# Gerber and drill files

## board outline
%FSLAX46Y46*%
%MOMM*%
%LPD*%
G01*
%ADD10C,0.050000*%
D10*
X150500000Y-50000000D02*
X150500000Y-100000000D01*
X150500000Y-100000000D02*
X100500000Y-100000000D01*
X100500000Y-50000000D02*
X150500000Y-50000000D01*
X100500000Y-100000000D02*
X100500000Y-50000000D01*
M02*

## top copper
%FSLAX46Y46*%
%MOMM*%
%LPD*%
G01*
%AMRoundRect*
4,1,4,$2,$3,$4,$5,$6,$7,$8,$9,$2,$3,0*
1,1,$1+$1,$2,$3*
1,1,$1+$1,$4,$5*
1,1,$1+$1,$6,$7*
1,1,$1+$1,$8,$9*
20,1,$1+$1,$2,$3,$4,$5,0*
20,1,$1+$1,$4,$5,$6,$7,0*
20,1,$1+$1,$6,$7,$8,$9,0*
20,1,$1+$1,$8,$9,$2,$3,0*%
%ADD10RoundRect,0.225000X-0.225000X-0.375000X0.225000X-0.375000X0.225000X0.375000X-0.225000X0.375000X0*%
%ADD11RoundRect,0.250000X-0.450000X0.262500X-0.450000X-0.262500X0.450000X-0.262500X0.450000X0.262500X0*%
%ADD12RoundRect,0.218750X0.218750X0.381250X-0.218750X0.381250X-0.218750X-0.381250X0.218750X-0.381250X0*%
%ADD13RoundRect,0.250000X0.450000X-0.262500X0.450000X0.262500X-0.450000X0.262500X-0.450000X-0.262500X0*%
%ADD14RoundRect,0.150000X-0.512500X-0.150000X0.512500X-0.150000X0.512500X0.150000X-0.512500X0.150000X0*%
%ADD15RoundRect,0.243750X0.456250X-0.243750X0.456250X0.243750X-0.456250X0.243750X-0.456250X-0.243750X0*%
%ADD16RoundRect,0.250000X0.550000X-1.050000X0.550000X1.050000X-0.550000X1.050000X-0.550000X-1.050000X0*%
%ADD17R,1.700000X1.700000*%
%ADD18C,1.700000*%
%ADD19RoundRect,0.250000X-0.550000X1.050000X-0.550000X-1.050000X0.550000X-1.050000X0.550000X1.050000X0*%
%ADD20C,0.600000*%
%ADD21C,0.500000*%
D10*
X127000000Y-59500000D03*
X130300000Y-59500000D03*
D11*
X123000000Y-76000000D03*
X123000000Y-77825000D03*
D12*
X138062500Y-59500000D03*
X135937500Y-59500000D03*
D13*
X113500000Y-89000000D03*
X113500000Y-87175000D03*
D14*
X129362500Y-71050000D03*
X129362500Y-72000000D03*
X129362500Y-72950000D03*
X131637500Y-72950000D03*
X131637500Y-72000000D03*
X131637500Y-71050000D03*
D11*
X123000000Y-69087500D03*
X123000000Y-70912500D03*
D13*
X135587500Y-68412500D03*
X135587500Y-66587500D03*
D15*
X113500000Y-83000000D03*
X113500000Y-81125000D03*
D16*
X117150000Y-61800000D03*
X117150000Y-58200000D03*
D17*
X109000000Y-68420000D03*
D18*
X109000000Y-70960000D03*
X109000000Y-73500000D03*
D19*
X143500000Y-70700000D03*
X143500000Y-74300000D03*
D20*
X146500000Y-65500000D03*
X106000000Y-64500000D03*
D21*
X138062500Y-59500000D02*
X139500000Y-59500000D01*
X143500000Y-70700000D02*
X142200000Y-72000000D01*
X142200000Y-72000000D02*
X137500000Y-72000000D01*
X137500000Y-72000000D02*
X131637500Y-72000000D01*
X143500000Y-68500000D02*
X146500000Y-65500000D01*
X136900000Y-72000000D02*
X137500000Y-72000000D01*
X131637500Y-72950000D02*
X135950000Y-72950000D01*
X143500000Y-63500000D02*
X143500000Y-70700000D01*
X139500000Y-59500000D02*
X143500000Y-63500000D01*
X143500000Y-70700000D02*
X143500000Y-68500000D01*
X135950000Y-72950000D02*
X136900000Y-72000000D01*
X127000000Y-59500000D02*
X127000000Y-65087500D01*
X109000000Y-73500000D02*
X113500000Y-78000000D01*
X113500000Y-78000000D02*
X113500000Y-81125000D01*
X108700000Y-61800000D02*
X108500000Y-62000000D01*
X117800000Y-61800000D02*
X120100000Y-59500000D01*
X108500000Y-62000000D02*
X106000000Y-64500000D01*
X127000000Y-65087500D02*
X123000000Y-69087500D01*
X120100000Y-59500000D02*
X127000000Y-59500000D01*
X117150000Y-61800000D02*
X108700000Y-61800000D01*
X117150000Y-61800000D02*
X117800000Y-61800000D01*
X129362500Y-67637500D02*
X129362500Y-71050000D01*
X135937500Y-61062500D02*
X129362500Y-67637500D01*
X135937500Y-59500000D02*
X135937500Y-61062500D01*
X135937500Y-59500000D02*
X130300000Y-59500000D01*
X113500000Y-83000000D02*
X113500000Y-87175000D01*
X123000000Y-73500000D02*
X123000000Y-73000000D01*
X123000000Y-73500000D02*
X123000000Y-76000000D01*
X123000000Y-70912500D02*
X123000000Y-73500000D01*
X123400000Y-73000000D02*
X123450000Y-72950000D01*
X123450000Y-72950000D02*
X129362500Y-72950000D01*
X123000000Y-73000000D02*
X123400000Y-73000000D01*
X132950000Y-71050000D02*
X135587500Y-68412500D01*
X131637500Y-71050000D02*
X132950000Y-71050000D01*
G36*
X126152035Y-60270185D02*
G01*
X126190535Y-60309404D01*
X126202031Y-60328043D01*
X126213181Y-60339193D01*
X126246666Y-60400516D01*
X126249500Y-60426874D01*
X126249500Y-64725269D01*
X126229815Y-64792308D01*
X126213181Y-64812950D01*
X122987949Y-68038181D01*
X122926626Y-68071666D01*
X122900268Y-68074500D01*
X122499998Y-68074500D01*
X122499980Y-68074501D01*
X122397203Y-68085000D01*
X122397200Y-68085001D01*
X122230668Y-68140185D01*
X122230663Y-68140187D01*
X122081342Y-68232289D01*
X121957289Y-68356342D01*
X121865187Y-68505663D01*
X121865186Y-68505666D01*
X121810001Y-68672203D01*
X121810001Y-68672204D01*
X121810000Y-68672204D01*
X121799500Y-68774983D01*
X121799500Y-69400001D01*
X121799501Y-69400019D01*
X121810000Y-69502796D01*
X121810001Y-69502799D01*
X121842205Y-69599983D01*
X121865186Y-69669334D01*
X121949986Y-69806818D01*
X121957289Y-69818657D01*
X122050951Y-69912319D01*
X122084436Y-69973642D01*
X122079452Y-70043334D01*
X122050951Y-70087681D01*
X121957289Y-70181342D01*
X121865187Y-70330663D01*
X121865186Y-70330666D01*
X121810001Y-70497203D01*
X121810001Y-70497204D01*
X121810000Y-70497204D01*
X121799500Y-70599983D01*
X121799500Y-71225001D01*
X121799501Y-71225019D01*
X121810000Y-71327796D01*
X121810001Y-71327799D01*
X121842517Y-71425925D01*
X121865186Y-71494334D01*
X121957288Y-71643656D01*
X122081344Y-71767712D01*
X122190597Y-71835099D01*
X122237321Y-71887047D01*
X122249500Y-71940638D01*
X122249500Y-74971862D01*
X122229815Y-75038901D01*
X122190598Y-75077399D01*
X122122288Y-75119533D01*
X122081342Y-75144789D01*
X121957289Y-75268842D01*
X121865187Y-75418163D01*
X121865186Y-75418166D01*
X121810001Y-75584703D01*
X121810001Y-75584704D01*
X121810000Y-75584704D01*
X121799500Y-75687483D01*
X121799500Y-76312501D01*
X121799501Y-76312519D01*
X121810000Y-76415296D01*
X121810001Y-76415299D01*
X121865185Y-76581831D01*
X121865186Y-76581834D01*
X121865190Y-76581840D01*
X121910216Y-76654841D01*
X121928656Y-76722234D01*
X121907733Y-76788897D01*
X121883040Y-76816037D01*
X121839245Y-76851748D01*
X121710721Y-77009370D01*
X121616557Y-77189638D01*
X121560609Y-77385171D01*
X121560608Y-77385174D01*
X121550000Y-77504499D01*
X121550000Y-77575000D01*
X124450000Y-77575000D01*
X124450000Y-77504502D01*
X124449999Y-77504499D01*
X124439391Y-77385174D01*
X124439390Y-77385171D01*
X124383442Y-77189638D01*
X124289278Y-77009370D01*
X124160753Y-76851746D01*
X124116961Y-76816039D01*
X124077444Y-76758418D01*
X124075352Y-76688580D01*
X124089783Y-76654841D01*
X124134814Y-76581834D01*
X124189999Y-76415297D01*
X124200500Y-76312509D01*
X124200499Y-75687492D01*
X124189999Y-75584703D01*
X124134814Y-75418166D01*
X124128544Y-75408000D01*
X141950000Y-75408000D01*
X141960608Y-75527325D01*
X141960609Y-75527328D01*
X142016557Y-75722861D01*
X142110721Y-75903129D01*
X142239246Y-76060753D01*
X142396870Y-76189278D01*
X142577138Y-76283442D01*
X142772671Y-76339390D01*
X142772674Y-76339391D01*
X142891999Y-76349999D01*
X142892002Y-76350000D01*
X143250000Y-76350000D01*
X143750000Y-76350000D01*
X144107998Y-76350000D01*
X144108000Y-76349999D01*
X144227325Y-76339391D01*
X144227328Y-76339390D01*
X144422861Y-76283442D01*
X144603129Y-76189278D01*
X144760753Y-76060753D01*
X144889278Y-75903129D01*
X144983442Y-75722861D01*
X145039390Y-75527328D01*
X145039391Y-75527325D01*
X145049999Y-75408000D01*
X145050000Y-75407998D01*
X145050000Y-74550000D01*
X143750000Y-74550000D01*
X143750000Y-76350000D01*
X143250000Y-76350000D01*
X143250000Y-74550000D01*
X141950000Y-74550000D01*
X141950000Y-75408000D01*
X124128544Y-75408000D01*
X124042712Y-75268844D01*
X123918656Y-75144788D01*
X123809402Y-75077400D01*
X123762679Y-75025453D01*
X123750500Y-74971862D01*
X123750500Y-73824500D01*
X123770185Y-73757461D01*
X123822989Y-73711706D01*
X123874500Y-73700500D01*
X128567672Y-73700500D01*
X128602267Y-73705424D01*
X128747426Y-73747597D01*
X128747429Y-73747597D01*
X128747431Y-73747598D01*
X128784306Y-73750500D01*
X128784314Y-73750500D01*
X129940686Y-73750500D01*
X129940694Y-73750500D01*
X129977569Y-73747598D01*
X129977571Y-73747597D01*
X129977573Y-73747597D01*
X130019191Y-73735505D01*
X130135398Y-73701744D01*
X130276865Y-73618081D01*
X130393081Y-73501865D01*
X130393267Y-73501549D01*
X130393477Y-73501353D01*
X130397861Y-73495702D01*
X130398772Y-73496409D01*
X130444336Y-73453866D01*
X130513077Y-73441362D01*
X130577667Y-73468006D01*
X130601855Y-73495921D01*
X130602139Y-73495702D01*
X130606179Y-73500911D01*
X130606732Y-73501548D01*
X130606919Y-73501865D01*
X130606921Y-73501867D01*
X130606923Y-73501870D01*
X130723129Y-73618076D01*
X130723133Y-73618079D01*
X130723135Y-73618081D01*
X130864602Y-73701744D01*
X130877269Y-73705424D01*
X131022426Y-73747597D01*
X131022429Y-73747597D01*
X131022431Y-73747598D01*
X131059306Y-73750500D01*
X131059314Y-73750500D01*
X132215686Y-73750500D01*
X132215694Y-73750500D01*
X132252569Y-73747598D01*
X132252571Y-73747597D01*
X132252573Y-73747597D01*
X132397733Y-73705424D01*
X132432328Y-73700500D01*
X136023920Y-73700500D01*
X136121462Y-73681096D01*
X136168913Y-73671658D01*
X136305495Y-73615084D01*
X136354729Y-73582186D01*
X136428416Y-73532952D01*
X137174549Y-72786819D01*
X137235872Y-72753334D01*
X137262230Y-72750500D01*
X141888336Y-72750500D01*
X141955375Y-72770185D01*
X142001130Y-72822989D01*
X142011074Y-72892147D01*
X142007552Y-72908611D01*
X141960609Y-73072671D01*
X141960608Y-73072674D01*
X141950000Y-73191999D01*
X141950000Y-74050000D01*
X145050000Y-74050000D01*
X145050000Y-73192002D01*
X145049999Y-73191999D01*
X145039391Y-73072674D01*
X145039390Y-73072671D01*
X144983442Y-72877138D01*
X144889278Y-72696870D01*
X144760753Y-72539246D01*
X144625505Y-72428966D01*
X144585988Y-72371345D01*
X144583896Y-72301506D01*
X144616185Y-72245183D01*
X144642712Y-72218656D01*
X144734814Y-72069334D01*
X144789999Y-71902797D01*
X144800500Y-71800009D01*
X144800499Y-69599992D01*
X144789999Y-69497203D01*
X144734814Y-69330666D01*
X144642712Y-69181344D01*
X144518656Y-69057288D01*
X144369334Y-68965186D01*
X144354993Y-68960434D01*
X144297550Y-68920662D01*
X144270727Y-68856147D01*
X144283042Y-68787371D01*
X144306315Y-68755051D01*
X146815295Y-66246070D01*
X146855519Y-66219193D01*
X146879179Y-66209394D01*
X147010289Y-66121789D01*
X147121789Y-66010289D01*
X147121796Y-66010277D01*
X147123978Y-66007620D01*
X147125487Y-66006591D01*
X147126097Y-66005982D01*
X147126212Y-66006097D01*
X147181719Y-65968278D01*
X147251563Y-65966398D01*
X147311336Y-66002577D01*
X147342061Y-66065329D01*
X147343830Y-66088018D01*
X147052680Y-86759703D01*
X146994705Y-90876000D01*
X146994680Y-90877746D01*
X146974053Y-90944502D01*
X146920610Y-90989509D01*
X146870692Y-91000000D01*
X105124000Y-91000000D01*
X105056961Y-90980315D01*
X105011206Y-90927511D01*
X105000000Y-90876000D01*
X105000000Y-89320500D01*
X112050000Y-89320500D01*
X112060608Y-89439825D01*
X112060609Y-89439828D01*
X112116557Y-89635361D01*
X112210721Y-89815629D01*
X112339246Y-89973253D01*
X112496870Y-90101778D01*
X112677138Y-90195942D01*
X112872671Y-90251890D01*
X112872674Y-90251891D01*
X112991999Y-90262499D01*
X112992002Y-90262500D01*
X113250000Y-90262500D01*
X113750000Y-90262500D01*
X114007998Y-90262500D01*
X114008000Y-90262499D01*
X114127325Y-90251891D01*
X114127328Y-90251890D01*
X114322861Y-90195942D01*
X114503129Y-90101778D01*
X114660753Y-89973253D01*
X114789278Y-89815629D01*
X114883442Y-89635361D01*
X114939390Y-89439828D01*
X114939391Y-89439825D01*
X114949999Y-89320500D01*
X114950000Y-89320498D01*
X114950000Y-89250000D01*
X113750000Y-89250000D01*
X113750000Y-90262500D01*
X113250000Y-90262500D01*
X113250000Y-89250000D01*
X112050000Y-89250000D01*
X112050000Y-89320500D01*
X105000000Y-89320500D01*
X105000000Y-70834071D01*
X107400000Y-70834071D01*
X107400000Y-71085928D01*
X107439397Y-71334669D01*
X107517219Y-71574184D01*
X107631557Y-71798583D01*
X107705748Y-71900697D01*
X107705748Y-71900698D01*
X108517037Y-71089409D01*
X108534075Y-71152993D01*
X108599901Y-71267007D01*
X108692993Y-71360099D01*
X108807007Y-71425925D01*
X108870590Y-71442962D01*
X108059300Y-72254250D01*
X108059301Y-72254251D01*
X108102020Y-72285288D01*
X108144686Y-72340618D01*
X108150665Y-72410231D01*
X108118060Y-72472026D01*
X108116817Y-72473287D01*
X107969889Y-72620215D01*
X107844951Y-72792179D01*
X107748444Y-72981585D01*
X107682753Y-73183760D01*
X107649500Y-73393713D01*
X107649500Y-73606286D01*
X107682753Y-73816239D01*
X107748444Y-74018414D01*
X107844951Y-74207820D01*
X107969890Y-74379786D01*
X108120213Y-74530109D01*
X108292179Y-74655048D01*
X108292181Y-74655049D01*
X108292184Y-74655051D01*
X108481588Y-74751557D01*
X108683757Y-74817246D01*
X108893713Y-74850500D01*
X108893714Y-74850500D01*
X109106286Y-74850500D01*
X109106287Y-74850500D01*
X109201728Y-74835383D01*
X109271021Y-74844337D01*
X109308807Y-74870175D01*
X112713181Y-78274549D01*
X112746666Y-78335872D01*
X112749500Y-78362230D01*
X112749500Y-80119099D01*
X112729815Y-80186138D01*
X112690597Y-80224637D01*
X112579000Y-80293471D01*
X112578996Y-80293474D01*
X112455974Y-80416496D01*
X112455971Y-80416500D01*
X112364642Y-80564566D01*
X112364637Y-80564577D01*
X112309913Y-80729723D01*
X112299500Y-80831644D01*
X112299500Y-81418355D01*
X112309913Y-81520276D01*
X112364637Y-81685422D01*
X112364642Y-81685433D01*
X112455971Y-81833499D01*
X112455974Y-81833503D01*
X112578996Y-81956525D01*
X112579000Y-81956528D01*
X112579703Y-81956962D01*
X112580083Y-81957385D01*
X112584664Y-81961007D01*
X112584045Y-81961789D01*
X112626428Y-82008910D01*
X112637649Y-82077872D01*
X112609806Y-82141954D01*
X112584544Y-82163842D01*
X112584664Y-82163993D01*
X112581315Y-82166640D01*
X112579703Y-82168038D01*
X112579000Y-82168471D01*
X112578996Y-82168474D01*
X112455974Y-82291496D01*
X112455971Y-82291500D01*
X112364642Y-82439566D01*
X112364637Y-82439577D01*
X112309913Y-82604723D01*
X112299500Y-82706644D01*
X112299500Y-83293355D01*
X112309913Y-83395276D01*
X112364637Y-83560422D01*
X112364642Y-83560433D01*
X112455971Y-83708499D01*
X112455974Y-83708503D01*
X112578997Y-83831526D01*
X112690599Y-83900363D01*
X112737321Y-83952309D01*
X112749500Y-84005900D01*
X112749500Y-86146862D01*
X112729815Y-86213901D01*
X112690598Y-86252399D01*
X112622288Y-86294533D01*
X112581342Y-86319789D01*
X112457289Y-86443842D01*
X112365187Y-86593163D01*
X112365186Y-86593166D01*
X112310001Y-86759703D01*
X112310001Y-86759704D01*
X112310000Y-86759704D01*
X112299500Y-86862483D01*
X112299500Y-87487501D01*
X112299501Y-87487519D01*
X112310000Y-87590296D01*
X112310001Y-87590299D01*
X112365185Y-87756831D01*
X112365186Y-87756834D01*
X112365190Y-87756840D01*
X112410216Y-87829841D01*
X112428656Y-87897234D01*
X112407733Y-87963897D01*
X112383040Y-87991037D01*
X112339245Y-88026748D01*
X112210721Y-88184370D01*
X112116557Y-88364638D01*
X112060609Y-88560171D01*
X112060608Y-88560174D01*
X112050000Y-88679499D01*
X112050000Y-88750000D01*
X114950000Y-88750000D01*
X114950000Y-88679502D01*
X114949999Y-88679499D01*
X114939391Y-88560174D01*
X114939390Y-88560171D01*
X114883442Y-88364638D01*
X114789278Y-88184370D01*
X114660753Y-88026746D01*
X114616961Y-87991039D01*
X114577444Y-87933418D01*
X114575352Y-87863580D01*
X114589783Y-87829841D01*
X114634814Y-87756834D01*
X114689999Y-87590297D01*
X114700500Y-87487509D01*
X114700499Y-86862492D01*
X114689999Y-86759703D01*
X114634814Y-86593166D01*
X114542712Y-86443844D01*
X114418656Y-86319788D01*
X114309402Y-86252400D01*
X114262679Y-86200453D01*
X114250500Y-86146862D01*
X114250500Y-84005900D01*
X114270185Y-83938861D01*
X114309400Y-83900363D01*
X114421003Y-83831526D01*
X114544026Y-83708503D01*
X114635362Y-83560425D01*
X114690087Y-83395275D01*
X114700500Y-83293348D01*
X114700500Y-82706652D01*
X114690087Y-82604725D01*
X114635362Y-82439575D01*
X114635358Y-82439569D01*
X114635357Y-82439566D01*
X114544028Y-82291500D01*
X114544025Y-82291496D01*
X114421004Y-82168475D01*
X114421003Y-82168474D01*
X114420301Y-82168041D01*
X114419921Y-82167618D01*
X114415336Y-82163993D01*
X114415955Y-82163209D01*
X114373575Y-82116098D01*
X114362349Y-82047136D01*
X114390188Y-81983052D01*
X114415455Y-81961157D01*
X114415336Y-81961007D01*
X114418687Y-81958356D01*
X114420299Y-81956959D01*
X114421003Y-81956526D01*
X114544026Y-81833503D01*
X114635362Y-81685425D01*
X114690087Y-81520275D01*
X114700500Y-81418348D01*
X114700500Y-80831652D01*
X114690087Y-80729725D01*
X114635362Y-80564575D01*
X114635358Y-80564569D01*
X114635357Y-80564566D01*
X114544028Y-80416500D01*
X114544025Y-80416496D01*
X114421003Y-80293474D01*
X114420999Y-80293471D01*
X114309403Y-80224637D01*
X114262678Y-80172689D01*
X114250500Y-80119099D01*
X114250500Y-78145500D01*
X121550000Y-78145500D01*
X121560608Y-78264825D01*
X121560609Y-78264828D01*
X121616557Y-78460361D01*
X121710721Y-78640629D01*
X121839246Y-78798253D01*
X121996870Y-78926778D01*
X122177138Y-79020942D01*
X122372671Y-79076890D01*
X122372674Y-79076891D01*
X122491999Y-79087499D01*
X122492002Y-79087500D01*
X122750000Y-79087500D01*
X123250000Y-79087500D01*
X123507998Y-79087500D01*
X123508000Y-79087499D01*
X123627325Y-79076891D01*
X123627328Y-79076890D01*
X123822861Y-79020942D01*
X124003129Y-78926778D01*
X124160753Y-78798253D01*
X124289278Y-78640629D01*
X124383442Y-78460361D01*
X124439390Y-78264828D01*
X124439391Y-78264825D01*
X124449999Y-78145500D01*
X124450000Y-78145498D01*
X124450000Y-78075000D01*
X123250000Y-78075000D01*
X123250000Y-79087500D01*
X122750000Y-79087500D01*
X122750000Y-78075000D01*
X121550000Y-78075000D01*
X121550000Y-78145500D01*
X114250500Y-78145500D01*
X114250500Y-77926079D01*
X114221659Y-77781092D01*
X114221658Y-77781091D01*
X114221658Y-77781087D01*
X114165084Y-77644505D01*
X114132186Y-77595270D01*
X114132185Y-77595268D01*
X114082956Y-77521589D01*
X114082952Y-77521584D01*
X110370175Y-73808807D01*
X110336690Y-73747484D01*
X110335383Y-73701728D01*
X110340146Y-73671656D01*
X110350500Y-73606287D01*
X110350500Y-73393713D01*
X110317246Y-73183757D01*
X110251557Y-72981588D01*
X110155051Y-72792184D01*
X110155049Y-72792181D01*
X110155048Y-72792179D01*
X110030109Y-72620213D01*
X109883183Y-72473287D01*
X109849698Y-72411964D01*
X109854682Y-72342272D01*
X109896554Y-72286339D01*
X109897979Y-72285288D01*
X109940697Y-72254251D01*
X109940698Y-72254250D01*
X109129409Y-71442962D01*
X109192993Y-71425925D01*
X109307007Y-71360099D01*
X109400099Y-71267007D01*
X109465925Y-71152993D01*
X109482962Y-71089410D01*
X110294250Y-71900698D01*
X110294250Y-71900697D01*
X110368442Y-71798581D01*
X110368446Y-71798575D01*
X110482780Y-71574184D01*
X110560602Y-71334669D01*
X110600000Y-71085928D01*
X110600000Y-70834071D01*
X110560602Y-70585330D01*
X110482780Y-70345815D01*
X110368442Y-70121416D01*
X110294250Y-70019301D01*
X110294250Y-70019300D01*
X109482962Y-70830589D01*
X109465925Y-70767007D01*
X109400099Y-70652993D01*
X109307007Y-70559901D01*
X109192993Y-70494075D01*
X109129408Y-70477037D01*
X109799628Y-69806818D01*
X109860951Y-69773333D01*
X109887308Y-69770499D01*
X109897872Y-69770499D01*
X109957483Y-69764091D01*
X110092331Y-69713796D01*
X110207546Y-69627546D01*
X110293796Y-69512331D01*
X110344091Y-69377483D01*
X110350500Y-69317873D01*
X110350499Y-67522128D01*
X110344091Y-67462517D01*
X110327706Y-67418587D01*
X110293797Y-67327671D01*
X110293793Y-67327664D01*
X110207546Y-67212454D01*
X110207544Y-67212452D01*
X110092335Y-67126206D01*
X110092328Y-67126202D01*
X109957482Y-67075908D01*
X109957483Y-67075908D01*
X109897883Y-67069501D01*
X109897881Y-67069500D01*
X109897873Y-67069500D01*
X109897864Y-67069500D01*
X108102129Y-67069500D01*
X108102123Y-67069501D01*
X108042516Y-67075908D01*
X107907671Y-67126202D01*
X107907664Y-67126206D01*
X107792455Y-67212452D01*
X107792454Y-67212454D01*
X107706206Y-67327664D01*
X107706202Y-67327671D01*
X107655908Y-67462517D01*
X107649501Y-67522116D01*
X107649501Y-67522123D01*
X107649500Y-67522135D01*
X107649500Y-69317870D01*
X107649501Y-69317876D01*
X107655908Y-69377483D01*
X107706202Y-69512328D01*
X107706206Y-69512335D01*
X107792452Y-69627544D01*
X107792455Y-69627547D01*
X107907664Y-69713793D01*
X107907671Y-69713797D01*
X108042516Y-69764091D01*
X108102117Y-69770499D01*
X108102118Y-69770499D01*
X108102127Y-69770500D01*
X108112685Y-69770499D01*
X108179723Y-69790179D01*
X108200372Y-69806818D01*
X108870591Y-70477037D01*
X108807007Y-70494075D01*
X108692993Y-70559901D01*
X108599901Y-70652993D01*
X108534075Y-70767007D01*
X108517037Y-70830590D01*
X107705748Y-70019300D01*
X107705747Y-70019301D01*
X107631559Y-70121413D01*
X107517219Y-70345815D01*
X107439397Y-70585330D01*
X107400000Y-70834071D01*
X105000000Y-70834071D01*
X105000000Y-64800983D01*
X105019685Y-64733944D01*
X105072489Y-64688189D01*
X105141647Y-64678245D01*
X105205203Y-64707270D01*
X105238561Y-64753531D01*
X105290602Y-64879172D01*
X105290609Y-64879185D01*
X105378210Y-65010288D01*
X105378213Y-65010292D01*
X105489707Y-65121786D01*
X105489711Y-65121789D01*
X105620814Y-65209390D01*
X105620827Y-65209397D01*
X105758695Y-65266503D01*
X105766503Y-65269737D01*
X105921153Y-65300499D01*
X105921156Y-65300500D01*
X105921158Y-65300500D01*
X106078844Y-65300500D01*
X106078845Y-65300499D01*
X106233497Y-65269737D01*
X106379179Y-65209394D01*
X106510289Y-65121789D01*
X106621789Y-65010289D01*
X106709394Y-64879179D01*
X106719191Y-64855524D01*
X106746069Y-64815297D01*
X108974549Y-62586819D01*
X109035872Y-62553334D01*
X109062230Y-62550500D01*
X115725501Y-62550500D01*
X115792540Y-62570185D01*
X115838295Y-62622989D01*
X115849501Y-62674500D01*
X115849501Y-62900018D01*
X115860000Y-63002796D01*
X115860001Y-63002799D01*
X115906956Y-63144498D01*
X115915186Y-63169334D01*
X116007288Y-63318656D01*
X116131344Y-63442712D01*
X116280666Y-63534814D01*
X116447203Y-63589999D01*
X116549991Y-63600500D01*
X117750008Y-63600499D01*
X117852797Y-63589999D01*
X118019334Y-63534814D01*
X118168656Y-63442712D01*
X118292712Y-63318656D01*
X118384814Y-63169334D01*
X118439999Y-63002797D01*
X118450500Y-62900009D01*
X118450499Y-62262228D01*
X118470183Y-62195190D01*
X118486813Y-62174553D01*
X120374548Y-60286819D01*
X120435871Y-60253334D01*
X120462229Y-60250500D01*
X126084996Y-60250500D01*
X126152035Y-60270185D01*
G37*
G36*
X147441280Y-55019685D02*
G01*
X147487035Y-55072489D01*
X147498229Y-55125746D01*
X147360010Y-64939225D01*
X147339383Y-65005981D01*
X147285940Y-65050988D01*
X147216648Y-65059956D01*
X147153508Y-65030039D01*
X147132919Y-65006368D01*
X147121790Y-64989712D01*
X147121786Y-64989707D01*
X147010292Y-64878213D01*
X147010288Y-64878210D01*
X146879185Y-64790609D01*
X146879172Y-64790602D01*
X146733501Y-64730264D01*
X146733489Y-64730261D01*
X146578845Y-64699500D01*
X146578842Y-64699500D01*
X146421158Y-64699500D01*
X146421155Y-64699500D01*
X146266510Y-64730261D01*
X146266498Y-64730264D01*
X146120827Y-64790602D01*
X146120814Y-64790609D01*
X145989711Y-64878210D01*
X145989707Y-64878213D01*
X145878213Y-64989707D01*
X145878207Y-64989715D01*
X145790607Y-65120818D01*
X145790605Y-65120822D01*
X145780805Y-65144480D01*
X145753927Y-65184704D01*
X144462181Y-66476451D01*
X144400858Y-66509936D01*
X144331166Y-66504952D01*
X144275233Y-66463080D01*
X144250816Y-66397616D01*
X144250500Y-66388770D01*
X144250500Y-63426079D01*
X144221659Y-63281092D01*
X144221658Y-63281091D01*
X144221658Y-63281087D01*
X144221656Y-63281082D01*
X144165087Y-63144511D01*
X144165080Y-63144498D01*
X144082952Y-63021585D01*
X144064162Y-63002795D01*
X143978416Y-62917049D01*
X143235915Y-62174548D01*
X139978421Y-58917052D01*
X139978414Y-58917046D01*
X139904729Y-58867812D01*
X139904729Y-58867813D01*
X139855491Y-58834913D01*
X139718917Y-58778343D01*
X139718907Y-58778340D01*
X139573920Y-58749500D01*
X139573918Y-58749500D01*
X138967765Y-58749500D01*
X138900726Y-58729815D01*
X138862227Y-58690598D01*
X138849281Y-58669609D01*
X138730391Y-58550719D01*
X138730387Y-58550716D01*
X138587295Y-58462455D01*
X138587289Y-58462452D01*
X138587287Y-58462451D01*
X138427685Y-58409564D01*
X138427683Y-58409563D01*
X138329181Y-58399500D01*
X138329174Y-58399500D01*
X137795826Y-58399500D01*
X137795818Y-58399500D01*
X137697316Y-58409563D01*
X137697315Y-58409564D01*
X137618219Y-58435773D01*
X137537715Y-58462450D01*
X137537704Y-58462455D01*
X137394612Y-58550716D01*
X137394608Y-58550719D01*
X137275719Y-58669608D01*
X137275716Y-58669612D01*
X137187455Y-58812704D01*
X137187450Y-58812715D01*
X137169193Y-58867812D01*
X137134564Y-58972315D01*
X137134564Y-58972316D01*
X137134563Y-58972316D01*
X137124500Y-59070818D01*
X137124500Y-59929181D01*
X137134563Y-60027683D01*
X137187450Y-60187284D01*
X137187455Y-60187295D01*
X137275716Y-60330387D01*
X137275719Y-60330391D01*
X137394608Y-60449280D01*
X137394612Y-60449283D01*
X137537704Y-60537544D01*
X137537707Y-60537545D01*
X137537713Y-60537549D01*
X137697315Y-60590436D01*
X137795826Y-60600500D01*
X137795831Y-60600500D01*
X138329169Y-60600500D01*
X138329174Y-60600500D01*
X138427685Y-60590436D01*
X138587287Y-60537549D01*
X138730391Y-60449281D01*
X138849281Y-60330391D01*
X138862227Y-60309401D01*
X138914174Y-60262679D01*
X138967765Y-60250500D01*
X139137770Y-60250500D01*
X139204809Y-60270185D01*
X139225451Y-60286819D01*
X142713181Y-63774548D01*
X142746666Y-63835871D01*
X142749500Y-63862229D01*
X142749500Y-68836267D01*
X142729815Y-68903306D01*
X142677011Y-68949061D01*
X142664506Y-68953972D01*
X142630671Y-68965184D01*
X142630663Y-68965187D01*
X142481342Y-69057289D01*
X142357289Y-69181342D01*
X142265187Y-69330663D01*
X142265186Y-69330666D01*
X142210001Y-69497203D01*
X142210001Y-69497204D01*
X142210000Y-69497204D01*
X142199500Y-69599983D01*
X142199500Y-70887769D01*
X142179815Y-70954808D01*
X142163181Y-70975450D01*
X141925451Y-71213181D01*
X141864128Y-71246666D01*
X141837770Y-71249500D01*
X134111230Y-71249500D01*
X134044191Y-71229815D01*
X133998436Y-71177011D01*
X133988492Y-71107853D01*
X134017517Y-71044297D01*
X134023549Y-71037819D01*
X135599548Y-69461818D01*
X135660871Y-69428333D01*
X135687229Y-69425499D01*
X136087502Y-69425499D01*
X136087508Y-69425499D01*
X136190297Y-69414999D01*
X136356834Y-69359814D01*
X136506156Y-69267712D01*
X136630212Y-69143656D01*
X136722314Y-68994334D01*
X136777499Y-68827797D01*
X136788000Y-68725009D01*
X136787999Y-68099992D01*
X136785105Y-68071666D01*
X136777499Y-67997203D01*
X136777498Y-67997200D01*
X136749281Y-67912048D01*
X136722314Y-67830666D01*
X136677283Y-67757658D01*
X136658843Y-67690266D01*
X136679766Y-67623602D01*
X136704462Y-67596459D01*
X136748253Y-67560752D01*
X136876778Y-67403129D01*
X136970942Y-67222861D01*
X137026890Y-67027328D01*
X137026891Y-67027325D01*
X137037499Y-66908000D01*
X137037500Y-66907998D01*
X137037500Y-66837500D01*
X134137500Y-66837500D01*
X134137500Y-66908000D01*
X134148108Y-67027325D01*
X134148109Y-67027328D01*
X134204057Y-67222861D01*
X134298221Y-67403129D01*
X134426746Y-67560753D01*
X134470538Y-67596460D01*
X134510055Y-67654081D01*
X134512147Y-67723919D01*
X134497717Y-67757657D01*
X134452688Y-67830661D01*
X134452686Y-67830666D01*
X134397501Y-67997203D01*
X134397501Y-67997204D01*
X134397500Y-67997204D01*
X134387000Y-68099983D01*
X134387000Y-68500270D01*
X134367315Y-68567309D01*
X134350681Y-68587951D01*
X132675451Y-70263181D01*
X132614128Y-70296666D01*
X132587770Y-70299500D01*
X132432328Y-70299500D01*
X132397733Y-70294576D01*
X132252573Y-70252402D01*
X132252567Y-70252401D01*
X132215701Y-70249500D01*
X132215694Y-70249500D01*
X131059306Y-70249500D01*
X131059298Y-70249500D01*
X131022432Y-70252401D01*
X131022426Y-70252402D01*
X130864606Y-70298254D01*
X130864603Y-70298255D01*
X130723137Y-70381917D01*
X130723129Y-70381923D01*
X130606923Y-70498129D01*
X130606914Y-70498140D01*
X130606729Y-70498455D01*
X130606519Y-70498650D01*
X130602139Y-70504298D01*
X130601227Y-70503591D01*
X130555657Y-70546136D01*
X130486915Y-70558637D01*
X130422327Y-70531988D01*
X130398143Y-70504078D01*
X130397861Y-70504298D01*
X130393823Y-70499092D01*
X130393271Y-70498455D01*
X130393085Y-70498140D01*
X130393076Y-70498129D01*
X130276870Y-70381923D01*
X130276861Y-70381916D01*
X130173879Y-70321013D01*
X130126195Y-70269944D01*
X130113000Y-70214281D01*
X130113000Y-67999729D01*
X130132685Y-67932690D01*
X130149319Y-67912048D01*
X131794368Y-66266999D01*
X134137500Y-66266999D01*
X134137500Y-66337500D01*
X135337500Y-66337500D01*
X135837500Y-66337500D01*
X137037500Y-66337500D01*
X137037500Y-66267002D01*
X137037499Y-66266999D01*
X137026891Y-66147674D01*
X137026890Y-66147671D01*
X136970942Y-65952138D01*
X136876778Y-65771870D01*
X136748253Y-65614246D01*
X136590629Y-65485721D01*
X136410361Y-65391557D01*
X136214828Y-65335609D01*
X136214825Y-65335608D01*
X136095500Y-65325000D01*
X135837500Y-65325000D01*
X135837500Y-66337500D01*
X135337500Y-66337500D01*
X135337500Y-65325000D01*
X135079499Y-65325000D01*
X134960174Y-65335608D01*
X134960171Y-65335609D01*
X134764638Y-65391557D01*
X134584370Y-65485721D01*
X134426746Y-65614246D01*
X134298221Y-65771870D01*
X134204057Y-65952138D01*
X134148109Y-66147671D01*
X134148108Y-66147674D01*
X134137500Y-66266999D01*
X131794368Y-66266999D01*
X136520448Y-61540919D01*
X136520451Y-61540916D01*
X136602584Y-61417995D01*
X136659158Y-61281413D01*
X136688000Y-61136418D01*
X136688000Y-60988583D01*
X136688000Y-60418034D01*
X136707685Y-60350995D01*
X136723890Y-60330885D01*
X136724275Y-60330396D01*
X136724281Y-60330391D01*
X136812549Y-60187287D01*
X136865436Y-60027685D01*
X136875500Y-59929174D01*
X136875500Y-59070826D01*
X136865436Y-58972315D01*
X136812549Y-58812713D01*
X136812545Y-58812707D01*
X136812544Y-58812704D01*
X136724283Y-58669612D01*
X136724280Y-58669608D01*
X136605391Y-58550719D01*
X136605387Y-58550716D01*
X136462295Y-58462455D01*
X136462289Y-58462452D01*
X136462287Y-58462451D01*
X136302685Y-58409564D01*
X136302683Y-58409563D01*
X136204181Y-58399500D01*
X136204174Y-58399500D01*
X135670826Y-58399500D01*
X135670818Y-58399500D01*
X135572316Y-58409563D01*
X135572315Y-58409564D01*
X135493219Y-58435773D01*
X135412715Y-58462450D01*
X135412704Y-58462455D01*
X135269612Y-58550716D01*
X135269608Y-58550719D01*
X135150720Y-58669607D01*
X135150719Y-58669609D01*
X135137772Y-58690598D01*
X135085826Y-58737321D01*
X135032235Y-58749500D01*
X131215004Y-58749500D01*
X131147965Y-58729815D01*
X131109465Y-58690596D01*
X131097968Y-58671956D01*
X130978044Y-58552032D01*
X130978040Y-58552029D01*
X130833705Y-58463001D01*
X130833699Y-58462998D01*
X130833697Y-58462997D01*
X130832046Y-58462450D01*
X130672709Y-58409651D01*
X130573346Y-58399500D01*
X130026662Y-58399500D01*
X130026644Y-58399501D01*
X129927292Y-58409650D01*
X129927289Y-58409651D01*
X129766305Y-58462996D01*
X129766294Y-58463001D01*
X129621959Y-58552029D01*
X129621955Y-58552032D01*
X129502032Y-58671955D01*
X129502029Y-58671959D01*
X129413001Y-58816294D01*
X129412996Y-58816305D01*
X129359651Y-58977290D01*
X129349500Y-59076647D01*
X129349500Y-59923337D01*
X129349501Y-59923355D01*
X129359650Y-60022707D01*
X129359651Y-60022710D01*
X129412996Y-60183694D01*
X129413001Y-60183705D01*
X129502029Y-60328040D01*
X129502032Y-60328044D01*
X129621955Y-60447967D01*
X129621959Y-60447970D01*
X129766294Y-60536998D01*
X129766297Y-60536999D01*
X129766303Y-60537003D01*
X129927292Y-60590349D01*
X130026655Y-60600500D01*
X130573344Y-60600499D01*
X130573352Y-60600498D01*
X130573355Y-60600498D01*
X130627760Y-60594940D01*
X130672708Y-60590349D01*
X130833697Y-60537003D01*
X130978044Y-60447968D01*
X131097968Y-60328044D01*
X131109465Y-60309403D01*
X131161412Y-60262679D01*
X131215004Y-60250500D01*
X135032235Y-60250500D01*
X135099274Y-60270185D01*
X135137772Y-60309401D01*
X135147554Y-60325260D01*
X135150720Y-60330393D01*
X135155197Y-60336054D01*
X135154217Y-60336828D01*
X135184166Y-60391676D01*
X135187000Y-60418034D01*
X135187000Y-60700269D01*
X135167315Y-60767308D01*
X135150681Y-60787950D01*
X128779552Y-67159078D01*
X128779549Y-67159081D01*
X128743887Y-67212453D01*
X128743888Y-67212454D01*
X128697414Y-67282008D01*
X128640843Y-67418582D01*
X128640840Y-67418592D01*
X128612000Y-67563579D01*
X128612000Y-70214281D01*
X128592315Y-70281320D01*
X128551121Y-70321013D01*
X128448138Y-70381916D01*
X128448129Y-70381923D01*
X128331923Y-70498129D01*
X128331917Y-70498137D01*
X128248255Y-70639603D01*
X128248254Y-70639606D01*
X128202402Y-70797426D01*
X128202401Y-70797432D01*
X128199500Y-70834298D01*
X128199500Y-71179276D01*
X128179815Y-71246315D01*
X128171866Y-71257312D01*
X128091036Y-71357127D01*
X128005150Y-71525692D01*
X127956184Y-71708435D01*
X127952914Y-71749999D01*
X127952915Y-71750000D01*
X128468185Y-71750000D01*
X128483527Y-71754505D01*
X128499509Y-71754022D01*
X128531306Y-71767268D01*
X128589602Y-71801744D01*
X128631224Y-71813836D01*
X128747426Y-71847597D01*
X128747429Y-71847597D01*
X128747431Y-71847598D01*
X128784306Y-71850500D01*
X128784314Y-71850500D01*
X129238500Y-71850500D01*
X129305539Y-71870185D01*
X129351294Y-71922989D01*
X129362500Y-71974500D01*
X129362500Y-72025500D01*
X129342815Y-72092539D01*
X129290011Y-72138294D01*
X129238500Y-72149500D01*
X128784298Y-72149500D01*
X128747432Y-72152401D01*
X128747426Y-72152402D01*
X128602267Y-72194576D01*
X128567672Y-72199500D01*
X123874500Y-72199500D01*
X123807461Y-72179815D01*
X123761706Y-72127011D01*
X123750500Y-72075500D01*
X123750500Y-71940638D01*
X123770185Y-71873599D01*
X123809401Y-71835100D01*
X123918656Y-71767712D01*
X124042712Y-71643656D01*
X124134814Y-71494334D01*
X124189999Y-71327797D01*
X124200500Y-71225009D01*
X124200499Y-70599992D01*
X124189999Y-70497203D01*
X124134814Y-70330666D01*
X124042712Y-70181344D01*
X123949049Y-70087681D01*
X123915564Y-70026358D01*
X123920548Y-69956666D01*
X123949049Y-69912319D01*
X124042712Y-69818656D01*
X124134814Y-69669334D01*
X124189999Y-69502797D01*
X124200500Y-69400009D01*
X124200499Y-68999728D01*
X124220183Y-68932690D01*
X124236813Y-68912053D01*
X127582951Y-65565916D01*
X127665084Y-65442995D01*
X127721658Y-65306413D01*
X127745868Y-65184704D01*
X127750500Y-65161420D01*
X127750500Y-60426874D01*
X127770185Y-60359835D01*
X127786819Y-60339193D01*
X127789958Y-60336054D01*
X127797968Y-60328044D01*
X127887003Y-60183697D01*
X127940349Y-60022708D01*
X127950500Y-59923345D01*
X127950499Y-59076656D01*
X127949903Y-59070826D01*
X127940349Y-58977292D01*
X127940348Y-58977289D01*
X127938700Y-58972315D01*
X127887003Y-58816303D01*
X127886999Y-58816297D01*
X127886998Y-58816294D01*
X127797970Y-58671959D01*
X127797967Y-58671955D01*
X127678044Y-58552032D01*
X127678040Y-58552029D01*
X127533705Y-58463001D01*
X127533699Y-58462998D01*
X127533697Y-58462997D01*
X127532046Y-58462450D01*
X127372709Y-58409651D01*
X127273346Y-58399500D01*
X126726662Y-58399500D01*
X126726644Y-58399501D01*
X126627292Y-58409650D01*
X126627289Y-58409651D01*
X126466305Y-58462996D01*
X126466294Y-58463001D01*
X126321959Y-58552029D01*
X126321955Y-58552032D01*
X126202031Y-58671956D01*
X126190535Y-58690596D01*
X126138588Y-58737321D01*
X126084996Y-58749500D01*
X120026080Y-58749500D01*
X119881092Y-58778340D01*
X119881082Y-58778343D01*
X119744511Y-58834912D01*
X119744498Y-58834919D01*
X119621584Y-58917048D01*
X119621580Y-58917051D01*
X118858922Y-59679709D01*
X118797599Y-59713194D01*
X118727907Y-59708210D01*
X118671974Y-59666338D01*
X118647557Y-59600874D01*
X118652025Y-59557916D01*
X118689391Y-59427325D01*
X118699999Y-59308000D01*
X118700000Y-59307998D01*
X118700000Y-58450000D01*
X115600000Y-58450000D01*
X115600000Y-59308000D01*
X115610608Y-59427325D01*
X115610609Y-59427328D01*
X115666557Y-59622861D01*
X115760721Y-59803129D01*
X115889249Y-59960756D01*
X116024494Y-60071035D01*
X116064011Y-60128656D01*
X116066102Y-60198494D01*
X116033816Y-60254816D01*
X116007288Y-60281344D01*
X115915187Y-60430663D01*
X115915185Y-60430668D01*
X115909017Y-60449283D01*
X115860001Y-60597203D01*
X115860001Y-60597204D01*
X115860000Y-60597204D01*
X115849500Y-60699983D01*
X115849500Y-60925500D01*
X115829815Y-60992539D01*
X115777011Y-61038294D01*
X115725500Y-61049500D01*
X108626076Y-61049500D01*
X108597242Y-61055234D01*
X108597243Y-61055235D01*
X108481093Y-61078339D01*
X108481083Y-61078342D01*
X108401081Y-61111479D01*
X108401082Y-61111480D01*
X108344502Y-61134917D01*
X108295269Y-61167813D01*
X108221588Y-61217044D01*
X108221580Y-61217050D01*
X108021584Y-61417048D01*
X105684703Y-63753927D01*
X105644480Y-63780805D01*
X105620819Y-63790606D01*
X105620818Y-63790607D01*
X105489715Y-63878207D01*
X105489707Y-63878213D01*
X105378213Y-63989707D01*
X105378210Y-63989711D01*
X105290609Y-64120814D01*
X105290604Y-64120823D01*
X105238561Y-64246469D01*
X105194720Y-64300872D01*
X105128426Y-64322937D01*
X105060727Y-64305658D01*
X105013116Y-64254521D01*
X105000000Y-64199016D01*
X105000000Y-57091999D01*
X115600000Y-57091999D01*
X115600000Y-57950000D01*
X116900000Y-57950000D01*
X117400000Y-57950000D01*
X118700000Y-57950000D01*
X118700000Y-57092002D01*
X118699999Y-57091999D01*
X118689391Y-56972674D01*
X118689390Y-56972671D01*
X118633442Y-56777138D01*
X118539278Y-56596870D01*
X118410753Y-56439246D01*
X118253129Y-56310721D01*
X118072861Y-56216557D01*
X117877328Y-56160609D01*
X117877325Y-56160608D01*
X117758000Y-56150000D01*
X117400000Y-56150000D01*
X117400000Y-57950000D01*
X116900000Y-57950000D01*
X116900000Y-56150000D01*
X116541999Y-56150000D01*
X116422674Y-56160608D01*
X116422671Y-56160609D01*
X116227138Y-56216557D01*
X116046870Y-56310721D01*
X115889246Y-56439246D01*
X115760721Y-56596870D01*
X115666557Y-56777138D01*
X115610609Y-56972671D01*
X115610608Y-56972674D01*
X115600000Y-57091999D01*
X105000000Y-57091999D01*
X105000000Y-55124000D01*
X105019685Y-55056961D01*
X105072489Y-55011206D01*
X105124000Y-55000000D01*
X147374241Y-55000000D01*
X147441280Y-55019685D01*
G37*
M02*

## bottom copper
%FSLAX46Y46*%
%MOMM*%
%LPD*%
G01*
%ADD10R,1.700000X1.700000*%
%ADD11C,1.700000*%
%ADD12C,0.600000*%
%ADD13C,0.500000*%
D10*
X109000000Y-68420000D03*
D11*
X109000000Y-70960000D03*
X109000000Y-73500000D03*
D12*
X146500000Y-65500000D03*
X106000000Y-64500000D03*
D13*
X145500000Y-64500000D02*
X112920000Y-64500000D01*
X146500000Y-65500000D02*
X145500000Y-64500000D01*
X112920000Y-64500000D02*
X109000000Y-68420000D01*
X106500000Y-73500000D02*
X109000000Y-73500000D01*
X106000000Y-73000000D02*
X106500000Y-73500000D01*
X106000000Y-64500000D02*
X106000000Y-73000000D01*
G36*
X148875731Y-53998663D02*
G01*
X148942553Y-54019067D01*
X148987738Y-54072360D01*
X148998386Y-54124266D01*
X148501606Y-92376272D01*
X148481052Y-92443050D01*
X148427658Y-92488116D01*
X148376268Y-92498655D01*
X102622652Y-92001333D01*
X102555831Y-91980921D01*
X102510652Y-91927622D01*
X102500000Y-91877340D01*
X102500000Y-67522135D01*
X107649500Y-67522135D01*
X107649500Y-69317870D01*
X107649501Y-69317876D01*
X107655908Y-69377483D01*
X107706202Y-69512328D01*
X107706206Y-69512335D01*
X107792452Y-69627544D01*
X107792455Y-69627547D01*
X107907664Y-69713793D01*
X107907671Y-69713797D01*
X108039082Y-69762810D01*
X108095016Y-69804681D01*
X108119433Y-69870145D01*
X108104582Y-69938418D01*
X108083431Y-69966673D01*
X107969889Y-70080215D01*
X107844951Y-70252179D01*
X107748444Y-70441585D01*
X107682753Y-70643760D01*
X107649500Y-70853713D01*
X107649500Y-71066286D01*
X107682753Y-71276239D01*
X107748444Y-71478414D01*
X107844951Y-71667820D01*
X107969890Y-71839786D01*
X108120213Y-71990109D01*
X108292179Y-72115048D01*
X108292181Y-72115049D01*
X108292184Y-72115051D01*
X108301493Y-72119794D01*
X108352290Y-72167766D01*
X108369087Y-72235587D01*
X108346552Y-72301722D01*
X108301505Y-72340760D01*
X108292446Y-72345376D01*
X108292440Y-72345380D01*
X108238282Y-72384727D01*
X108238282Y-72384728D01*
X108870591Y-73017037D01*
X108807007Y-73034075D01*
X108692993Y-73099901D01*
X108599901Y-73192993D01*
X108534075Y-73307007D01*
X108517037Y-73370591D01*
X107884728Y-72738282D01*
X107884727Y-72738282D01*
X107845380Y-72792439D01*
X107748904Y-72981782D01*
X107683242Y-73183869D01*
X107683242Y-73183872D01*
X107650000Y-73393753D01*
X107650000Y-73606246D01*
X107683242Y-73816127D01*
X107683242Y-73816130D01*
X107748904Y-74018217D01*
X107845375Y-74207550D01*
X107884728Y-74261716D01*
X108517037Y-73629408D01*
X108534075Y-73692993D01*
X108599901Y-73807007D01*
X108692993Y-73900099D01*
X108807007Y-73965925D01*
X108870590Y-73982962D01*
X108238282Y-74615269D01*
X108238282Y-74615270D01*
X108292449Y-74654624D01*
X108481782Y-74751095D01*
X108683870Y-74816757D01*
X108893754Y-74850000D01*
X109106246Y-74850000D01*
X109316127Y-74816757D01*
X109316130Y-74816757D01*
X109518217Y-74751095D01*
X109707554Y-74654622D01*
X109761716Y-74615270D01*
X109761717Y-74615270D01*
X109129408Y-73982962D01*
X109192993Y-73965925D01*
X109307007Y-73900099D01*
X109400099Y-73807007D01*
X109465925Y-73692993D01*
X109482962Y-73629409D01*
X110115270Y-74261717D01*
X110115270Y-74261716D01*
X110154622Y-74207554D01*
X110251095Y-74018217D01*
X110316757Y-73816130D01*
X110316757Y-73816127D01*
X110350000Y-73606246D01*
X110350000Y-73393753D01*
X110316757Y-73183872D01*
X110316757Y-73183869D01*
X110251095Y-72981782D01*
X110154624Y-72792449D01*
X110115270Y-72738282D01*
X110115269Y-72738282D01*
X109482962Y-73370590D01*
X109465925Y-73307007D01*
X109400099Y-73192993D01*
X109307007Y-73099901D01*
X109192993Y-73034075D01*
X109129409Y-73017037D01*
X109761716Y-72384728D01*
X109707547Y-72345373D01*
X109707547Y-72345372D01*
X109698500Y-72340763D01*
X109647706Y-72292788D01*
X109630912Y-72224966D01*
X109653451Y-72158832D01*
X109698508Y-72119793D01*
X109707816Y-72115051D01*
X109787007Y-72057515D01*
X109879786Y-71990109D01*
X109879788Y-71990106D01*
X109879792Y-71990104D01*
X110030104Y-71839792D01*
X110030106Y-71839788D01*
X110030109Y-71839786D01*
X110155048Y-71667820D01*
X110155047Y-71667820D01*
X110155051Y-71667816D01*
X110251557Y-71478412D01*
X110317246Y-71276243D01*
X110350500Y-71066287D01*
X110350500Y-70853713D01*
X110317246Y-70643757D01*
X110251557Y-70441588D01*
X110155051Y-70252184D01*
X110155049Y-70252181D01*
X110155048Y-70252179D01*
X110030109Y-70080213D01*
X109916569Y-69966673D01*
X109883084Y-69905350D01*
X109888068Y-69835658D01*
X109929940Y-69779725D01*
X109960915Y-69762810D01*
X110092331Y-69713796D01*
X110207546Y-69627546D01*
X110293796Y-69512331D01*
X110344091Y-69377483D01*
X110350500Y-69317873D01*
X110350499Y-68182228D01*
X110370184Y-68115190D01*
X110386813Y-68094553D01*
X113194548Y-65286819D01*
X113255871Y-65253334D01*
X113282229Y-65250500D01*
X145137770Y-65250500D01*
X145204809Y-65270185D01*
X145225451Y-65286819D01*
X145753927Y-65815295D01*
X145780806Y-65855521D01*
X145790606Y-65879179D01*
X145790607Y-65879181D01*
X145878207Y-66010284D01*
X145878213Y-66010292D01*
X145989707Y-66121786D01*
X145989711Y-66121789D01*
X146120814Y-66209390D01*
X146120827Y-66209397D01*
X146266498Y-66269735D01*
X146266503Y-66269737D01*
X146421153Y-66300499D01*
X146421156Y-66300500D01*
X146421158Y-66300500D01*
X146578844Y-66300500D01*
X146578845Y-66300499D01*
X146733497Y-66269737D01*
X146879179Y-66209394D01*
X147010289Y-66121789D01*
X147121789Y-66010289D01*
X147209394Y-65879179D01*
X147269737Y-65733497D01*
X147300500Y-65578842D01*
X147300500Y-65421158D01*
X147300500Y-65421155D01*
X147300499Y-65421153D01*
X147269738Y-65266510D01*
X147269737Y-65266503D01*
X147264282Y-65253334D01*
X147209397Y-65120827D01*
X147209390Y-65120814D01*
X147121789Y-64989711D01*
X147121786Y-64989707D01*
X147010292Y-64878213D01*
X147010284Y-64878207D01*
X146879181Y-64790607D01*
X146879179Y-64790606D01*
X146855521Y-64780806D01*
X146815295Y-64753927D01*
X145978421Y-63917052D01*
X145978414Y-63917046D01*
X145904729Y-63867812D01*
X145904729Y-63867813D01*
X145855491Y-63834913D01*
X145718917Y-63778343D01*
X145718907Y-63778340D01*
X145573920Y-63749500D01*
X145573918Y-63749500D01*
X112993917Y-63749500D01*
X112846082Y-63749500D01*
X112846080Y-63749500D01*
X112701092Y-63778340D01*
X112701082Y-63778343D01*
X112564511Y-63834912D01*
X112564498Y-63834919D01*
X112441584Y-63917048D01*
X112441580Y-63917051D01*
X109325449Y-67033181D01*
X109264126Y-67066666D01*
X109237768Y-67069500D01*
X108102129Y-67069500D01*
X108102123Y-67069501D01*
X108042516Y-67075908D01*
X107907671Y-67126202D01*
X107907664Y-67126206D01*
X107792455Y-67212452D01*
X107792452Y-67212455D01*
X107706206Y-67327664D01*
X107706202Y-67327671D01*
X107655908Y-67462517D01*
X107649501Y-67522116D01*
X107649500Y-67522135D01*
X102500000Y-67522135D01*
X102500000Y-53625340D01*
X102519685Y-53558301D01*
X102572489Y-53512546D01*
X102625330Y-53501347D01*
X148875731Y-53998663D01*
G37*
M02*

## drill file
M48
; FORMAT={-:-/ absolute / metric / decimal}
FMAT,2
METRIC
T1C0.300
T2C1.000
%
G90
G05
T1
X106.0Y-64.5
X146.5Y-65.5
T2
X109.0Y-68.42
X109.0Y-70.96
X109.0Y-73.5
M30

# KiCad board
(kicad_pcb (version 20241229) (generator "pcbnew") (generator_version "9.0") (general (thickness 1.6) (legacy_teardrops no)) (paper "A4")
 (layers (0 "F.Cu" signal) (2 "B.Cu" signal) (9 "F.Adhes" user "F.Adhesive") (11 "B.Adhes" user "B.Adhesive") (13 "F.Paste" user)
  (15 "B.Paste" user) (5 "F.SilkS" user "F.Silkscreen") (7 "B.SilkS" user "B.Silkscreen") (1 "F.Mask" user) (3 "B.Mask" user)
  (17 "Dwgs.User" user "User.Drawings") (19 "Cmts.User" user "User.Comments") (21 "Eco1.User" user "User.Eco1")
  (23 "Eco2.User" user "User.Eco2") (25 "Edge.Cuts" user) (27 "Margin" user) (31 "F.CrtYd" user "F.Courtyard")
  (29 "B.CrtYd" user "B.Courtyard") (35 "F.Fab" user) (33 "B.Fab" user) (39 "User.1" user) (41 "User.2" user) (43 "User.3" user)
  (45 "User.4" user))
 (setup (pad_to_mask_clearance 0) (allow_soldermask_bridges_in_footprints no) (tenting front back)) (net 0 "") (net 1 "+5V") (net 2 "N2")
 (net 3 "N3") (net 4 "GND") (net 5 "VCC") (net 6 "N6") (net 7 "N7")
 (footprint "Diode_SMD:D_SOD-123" (layer "F.Cu") (at 128.65 59.5)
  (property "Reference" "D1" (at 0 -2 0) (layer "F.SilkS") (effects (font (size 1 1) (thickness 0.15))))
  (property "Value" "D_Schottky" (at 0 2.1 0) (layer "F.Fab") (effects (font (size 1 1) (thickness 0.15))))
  (pad "1" smd roundrect (at -1.65 0) (size 0.9 1.2) (layers "F.Cu" "F.Mask" "F.Paste") (roundrect_rratio 0.25) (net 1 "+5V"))
  (pad "2" smd roundrect (at 1.65 0) (size 0.9 1.2) (layers "F.Cu" "F.Mask" "F.Paste") (roundrect_rratio 0.25) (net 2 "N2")))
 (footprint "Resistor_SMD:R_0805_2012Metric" (layer "F.Cu") (at 123 76.9125 -90)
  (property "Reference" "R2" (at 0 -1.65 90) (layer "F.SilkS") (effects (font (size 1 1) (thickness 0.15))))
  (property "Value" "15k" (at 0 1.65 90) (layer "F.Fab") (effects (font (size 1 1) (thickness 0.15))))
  (pad "1" smd roundrect (at -0.9125 0 270) (size 1.025 1.4) (layers "F.Cu" "F.Mask" "F.Paste") (roundrect_rratio 0.243902) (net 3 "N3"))
  (pad "2" smd roundrect (at 0.9125 0 270) (size 1.025 1.4) (layers "F.Cu" "F.Mask" "F.Paste") (roundrect_rratio 0.243902) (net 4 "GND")))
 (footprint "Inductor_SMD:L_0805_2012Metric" (layer "F.Cu") (at 137 59.5 180)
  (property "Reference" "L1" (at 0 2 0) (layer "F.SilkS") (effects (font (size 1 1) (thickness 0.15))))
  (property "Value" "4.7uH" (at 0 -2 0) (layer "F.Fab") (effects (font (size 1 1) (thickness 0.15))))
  (pad "1" smd roundrect (at -1.0625 0 180) (size 0.875 1.2) (layers "F.Cu" "F.Mask" "F.Paste") (roundrect_rratio 0.25) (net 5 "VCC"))
  (pad "2" smd roundrect (at 1.0625 0 180) (size 0.875 1.2) (layers "F.Cu" "F.Mask" "F.Paste") (roundrect_rratio 0.25) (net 2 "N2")))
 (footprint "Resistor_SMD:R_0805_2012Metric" (layer "F.Cu") (at 113.5 88.0875 90)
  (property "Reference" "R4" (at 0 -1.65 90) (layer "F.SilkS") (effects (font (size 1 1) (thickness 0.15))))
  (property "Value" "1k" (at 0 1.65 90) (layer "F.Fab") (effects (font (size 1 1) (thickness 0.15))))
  (pad "1" smd roundrect (at -0.9125 0 90) (size 1.025 1.4) (layers "F.Cu" "F.Mask" "F.Paste") (roundrect_rratio 0.243902) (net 4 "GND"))
  (pad "2" smd roundrect (at 0.9125 0 90) (size 1.025 1.4) (layers "F.Cu" "F.Mask" "F.Paste") (roundrect_rratio 0.243902) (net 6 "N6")))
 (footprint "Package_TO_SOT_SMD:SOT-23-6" (layer "F.Cu") (at 130.5 72)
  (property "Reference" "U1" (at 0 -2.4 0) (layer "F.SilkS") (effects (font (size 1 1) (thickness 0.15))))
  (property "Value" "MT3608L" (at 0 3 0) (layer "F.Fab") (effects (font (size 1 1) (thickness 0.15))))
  (pad "1" smd roundrect (at -1.1375 -0.95) (size 1.325 0.6) (layers "F.Cu" "F.Mask" "F.Paste") (roundrect_rratio 0.25) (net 2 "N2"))
  (pad "2" smd roundrect (at -1.1375 0) (size 1.325 0.6) (layers "F.Cu" "F.Mask" "F.Paste") (roundrect_rratio 0.25) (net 4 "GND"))
  (pad "3" smd roundrect (at -1.1375 0.95) (size 1.325 0.6) (layers "F.Cu" "F.Mask" "F.Paste") (roundrect_rratio 0.25) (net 3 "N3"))
  (pad "4" smd roundrect (at 1.1375 0.95) (size 1.325 0.6) (layers "F.Cu" "F.Mask" "F.Paste") (roundrect_rratio 0.25) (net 5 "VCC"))
  (pad "5" smd roundrect (at 1.1375 0) (size 1.325 0.6) (layers "F.Cu" "F.Mask" "F.Paste") (roundrect_rratio 0.25) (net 5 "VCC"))
  (pad "6" smd roundrect (at 1.1375 -0.95) (size 1.325 0.6) (layers "F.Cu" "F.Mask" "F.Paste") (roundrect_rratio 0.25) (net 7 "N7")))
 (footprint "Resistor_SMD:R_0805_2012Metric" (layer "F.Cu") (at 123 70 -90)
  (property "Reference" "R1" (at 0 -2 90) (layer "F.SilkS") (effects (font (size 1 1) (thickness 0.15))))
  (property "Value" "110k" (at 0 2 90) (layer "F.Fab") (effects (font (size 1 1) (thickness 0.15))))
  (pad "1" smd roundrect (at -0.9125 0 270) (size 1.025 1.4) (layers "F.Cu" "F.Mask" "F.Paste") (roundrect_rratio 0.243902) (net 1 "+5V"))
  (pad "2" smd roundrect (at 0.9125 0 270) (size 1.025 1.4) (layers "F.Cu" "F.Mask" "F.Paste") (roundrect_rratio 0.243902) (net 3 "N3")))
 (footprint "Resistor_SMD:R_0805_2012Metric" (layer "F.Cu") (at 135.5875 67.5 90)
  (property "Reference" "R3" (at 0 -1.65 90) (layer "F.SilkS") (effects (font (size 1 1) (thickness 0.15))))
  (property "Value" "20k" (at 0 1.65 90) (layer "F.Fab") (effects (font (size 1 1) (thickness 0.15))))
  (pad "1" smd roundrect (at -0.9125 0 90) (size 1.025 1.4) (layers "F.Cu" "F.Mask" "F.Paste") (roundrect_rratio 0.243902) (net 7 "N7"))
  (pad "2" smd roundrect (at 0.9125 0 90) (size 1.025 1.4) (layers "F.Cu" "F.Mask" "F.Paste") (roundrect_rratio 0.243902) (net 4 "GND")))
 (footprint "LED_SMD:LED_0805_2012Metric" (layer "F.Cu") (at 113.5 82.0625 90)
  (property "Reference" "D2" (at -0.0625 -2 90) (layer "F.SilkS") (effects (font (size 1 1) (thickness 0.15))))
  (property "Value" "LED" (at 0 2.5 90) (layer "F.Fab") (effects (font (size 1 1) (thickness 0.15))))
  (pad "1" smd roundrect (at -0.9375 0 90) (size 0.975 1.4) (layers "F.Cu" "F.Mask" "F.Paste") (roundrect_rratio 0.25) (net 6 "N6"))
  (pad "2" smd roundrect (at 0.9375 0 90) (size 0.975 1.4) (layers "F.Cu" "F.Mask" "F.Paste") (roundrect_rratio 0.25) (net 1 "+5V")))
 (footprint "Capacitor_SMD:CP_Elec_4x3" (layer "F.Cu") (at 117.15 60 90)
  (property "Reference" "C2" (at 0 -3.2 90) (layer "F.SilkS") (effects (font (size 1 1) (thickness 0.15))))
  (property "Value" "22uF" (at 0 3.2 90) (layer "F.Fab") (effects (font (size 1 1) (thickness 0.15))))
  (pad "1" smd roundrect (at -1.8 0 90) (size 2.6 1.6) (layers "F.Cu" "F.Mask" "F.Paste") (roundrect_rratio 0.15625) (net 1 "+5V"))
  (pad "2" smd roundrect (at 1.8 0 90) (size 2.6 1.6) (layers "F.Cu" "F.Mask" "F.Paste") (roundrect_rratio 0.15625) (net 4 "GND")))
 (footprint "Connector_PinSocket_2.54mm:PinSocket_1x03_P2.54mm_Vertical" (layer "F.Cu") (at 109 68.42)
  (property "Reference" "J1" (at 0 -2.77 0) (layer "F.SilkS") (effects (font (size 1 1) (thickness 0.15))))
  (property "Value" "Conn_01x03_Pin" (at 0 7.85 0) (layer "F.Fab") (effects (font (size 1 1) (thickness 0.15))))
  (pad "1" thru_hole rect (at 0 0) (size 1.7 1.7) (drill 1) (layers "*.Cu" "*.Mask") (remove_unused_layers no) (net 5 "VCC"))
  (pad "2" thru_hole circle (at 0 2.54) (size 1.7 1.7) (drill 1) (layers "*.Cu" "*.Mask") (remove_unused_layers no) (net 4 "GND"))
  (pad "3" thru_hole circle (at 0 5.08) (size 1.7 1.7) (drill 1) (layers "*.Cu" "*.Mask") (remove_unused_layers no) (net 1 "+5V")))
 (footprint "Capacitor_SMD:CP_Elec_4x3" (layer "F.Cu") (at 143.5 72.5 -90)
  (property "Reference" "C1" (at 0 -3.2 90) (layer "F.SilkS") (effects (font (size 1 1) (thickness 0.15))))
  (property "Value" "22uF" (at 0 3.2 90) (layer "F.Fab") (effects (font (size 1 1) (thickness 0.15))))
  (pad "1" smd roundrect (at -1.8 0 270) (size 2.6 1.6) (layers "F.Cu" "F.Mask" "F.Paste") (roundrect_rratio 0.15625) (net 5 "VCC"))
  (pad "2" smd roundrect (at 1.8 0 270) (size 2.6 1.6) (layers "F.Cu" "F.Mask" "F.Paste") (roundrect_rratio 0.15625) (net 4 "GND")))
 (gr_line (start 150.5 50) (end 150.5 100) (stroke (width 0.05) (type default)) (layer "Edge.Cuts"))
 (gr_line (start 150.5 100) (end 100.5 100) (stroke (width 0.05) (type default)) (layer "Edge.Cuts"))
 (gr_line (start 100.5 50) (end 150.5 50) (stroke (width 0.05) (type default)) (layer "Edge.Cuts"))
 (gr_line (start 100.5 100) (end 100.5 50) (stroke (width 0.05) (type default)) (layer "Edge.Cuts"))
 (segment (start 138.0625 59.5) (end 139.5 59.5) (width 0.5) (layer "F.Cu") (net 5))
 (segment (start 143.5 70.7) (end 142.2 72) (width 0.5) (layer "F.Cu") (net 5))
 (segment (start 142.2 72) (end 137.5 72) (width 0.5) (layer "F.Cu") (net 5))
 (segment (start 137.5 72) (end 131.6375 72) (width 0.5) (layer "F.Cu") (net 5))
 (segment (start 143.5 68.5) (end 146.5 65.5) (width 0.5) (layer "F.Cu") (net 5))
 (segment (start 136.9 72) (end 137.5 72) (width 0.5) (layer "F.Cu") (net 5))
 (segment (start 131.6375 72.95) (end 135.95 72.95) (width 0.5) (layer "F.Cu") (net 5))
 (segment (start 143.5 63.5) (end 143.5 70.7) (width 0.5) (layer "F.Cu") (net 5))
 (segment (start 139.5 59.5) (end 143.5 63.5) (width 0.5) (layer "F.Cu") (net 5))
 (segment (start 143.5 70.7) (end 143.5 68.5) (width 0.5) (layer "F.Cu") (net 5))
 (segment (start 135.95 72.95) (end 136.9 72) (width 0.5) (layer "F.Cu") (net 5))
 (via (at 146.5 65.5) (size 0.6) (drill 0.3) (layers "F.Cu" "B.Cu") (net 5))
 (segment (start 145.5 64.5) (end 112.92 64.5) (width 0.5) (layer "B.Cu") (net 5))
 (segment (start 146.5 65.5) (end 145.5 64.5) (width 0.5) (layer "B.Cu") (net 5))
 (segment (start 112.92 64.5) (end 109 68.42) (width 0.5) (layer "B.Cu") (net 5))
 (segment (start 127 59.5) (end 127 65.0875) (width 0.5) (layer "F.Cu") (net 1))
 (segment (start 109 73.5) (end 113.5 78) (width 0.5) (layer "F.Cu") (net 1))
 (segment (start 113.5 78) (end 113.5 81.125) (width 0.5) (layer "F.Cu") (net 1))
 (segment (start 108.7 61.8) (end 108.5 62) (width 0.5) (layer "F.Cu") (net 1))
 (segment (start 117.8 61.8) (end 120.1 59.5) (width 0.5) (layer "F.Cu") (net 1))
 (segment (start 108.5 62) (end 106 64.5) (width 0.5) (layer "F.Cu") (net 1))
 (segment (start 127 65.0875) (end 123 69.0875) (width 0.5) (layer "F.Cu") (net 1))
 (segment (start 120.1 59.5) (end 127 59.5) (width 0.5) (layer "F.Cu") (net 1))
 (segment (start 117.15 61.8) (end 108.7 61.8) (width 0.5) (layer "F.Cu") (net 1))
 (segment (start 117.15 61.8) (end 117.8 61.8) (width 0.5) (layer "F.Cu") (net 1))
 (via (at 106 64.5) (size 0.6) (drill 0.3) (layers "F.Cu" "B.Cu") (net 1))
 (segment (start 106.5 73.5) (end 109 73.5) (width 0.5) (layer "B.Cu") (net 1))
 (segment (start 106 73) (end 106.5 73.5) (width 0.5) (layer "B.Cu") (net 1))
 (segment (start 106 64.5) (end 106 73) (width 0.5) (layer "B.Cu") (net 1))
 (segment (start 129.3625 67.6375) (end 129.3625 71.05) (width 0.5) (layer "F.Cu") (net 2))
 (segment (start 135.9375 61.0625) (end 129.3625 67.6375) (width 0.5) (layer "F.Cu") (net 2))
 (segment (start 135.9375 59.5) (end 135.9375 61.0625) (width 0.5) (layer "F.Cu") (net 2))
 (segment (start 135.9375 59.5) (end 130.3 59.5) (width 0.5) (layer "F.Cu") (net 2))
 (segment (start 113.5 83) (end 113.5 87.175) (width 0.5) (layer "F.Cu") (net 6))
 (segment (start 123 73.5) (end 123 73) (width 0.5) (layer "F.Cu") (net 3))
 (segment (start 123 73.5) (end 123 76) (width 0.5) (layer "F.Cu") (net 3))
 (segment (start 123 70.9125) (end 123 73.5) (width 0.5) (layer "F.Cu") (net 3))
 (segment (start 123.4 73) (end 123.45 72.95) (width 0.5) (layer "F.Cu") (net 3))
 (segment (start 123.45 72.95) (end 129.3625 72.95) (width 0.5) (layer "F.Cu") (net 3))
 (segment (start 123 73) (end 123.4 73) (width 0.5) (layer "F.Cu") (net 3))
 (segment (start 132.95 71.05) (end 135.5875 68.4125) (width 0.5) (layer "F.Cu") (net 7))
 (segment (start 131.6375 71.05) (end 132.95 71.05) (width 0.5) (layer "F.Cu") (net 7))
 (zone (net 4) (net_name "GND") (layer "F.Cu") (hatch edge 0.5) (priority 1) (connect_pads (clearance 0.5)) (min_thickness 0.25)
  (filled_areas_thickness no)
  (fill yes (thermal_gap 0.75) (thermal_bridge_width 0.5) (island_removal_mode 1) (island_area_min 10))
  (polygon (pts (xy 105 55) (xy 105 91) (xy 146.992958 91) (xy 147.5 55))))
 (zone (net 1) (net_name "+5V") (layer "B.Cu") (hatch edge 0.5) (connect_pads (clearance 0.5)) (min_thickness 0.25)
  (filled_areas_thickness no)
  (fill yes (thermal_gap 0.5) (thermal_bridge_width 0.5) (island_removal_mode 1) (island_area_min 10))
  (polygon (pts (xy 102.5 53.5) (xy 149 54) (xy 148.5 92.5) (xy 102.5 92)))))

